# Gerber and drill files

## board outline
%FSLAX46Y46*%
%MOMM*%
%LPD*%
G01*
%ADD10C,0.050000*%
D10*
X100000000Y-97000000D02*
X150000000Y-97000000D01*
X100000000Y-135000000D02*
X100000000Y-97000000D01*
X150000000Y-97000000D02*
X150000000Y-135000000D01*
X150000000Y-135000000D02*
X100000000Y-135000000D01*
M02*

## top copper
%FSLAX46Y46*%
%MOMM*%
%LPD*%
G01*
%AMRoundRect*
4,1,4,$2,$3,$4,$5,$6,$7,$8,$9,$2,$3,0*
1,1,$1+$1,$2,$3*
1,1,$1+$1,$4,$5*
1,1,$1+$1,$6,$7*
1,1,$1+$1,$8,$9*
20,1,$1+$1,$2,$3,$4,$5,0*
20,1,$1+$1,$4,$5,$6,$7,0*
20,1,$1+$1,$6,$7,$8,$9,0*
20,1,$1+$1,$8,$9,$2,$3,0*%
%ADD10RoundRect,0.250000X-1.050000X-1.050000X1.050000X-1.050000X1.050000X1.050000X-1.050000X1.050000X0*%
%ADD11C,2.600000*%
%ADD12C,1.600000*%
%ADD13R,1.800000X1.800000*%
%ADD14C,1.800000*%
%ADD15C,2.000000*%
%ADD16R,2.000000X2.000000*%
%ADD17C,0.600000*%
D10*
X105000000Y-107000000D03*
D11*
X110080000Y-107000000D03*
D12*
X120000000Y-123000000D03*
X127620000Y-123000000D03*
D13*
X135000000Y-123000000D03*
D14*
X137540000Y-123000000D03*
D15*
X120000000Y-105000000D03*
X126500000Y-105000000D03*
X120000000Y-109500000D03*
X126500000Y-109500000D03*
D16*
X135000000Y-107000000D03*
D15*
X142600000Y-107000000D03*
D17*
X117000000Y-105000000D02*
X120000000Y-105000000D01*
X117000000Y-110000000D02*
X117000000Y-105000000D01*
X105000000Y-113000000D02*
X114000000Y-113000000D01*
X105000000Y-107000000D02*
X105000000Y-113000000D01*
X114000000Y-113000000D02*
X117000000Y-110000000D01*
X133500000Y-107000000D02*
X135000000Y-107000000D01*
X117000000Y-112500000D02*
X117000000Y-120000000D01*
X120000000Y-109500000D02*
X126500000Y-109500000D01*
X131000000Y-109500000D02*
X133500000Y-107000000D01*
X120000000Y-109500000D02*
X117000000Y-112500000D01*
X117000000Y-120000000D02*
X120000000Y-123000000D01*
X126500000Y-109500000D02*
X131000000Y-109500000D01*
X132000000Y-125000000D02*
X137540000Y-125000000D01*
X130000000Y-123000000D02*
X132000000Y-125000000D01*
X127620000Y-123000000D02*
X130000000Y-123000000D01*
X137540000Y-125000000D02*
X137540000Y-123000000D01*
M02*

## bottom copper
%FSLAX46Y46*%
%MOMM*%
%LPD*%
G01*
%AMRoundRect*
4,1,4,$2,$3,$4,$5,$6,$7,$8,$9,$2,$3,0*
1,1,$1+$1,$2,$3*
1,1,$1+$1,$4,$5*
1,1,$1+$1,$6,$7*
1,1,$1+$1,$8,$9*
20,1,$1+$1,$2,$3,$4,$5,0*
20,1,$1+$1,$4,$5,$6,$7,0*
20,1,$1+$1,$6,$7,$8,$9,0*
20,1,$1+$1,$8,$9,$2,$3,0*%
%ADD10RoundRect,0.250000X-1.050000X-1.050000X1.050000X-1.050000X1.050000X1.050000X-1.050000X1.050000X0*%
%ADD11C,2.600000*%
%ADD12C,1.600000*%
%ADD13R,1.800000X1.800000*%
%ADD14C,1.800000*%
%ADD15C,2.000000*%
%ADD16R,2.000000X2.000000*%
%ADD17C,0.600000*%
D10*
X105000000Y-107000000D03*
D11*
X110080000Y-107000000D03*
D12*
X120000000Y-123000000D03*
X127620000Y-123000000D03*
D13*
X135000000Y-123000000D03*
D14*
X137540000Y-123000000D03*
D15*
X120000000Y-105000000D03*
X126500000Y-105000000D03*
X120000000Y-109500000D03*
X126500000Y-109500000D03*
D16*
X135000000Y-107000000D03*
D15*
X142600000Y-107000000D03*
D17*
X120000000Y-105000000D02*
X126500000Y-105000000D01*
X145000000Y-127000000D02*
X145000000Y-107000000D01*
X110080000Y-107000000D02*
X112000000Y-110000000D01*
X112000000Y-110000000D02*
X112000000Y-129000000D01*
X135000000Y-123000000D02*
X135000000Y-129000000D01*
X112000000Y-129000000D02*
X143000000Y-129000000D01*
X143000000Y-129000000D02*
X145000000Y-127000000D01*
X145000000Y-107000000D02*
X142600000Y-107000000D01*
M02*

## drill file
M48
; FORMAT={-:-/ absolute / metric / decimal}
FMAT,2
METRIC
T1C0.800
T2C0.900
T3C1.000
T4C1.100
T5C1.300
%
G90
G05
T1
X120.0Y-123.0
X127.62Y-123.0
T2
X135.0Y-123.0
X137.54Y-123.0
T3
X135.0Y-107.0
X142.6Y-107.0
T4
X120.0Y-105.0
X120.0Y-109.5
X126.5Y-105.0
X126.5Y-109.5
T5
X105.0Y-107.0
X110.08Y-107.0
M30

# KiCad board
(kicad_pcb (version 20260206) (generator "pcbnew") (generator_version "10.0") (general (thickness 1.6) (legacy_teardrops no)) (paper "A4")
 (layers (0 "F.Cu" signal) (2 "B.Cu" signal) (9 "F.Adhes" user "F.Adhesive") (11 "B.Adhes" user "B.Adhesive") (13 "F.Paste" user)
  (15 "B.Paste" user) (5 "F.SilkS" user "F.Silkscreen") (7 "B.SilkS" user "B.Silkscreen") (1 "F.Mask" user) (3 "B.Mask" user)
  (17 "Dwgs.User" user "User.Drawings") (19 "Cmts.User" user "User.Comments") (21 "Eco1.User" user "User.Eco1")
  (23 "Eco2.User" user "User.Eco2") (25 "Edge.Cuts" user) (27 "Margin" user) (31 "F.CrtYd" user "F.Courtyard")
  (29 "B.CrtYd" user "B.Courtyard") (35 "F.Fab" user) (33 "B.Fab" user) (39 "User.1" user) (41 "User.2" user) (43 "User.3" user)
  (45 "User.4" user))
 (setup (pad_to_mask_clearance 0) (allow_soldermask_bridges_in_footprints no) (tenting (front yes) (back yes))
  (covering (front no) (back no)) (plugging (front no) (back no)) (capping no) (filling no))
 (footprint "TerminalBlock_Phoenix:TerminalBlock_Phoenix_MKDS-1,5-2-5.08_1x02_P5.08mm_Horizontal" (layer "F.Cu") (at 105 107)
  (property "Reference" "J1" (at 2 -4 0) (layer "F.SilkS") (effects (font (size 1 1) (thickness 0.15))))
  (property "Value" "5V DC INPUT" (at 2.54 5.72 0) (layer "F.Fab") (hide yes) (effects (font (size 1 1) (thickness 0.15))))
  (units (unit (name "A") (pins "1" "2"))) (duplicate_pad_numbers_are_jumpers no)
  (pad "1" thru_hole roundrect (at 0 0) (size 2.6 2.6) (drill 1.3) (layers "*.Cu" "*.Mask") (remove_unused_layers no)
   (roundrect_rratio 0.096154) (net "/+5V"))
  (pad "2" thru_hole circle (at 5.08 0) (size 2.6 2.6) (drill 1.3) (layers "*.Cu" "*.Mask") (remove_unused_layers no) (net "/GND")))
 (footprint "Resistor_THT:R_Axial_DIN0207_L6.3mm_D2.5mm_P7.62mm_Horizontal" (layer "F.Cu") (at 120 123)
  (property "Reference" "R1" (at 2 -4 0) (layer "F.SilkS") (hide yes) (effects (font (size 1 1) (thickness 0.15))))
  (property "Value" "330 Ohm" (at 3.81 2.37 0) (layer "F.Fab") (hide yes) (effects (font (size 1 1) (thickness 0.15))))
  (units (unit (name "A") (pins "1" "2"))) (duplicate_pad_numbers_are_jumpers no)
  (pad "1" thru_hole circle (at 0 0) (size 1.6 1.6) (drill 0.8) (layers "*.Cu" "*.Mask") (remove_unused_layers no) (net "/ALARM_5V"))
  (pad "2" thru_hole circle (at 7.62 0) (size 1.6 1.6) (drill 0.8) (layers "*.Cu" "*.Mask") (remove_unused_layers no) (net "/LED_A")))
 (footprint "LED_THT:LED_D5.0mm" (layer "F.Cu") (at 135 123)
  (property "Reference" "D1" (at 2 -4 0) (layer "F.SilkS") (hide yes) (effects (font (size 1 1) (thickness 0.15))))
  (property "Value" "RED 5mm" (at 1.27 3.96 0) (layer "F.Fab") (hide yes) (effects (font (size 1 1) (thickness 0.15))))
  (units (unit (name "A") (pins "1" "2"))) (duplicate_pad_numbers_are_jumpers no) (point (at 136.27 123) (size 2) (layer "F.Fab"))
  (pad "1" thru_hole rect (at 0 0) (size 1.8 1.8) (drill 0.9) (layers "*.Cu" "*.Mask") (remove_unused_layers no) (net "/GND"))
  (pad "2" thru_hole circle (at 2.54 0) (size 1.8 1.8) (drill 0.9) (layers "*.Cu" "*.Mask") (remove_unused_layers no) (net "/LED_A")))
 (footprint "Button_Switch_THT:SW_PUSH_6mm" (layer "F.Cu") (at 120 105)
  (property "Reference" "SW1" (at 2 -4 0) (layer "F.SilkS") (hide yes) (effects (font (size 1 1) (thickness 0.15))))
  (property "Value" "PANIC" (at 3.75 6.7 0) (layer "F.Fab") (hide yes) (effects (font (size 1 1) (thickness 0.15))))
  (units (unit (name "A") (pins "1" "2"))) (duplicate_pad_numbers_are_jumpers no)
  (pad "1" thru_hole circle (at 0 0 90) (size 2 2) (drill 1.1) (layers "*.Cu" "*.Mask") (remove_unused_layers no) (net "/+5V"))
  (pad "1" thru_hole circle (at 6.5 0 90) (size 2 2) (drill 1.1) (layers "*.Cu" "*.Mask") (remove_unused_layers no) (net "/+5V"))
  (pad "2" thru_hole circle (at 0 4.5 90) (size 2 2) (drill 1.1) (layers "*.Cu" "*.Mask") (remove_unused_layers no) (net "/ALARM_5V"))
  (pad "2" thru_hole circle (at 6.5 4.5 90) (size 2 2) (drill 1.1) (layers "*.Cu" "*.Mask") (remove_unused_layers no) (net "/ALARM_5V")))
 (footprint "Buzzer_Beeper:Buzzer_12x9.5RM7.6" (layer "F.Cu") (at 135 107)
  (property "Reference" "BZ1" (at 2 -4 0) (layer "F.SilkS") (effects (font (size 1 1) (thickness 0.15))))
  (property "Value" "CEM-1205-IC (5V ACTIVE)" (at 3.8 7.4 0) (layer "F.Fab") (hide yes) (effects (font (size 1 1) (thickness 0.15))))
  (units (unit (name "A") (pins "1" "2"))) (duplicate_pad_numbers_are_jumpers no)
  (pad "1" thru_hole rect (at 0 0) (size 2 2) (drill 1) (layers "*.Cu" "*.Mask") (remove_unused_layers no) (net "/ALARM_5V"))
  (pad "2" thru_hole circle (at 7.6 0) (size 2 2) (drill 1) (layers "*.Cu" "*.Mask") (remove_unused_layers no) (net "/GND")))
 (gr_line (start 100 97) (end 150 97) (stroke (width 0.05) (type default)) (layer "Edge.Cuts"))
 (gr_line (start 100 135) (end 100 97) (stroke (width 0.05) (type default)) (layer "Edge.Cuts"))
 (gr_line (start 150 97) (end 150 135) (stroke (width 0.05) (type default)) (layer "Edge.Cuts"))
 (gr_line (start 150 135) (end 100 135) (stroke (width 0.05) (type default)) (layer "Edge.Cuts"))
 (segment (start 117 105) (end 120 105) (width 0.6) (layer "F.Cu") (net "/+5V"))
 (segment (start 117 110) (end 117 105) (width 0.6) (layer "F.Cu") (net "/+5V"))
 (segment (start 105 113) (end 114 113) (width 0.6) (layer "F.Cu") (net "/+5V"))
 (segment (start 105 107) (end 105 113) (width 0.6) (layer "F.Cu") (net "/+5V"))
 (segment (start 114 113) (end 117 110) (width 0.6) (layer "F.Cu") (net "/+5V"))
 (segment (start 120 105) (end 126.5 105) (width 0.6) (layer "B.Cu") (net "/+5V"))
 (segment (start 145 127) (end 145 107) (width 0.6) (layer "B.Cu") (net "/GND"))
 (segment (start 110.08 107) (end 112 110) (width 0.6) (layer "B.Cu") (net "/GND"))
 (segment (start 112 110) (end 112 129) (width 0.6) (layer "B.Cu") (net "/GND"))
 (segment (start 135 123) (end 135 129) (width 0.6) (layer "B.Cu") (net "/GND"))
 (segment (start 112 129) (end 143 129) (width 0.6) (layer "B.Cu") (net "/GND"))
 (segment (start 143 129) (end 145 127) (width 0.6) (layer "B.Cu") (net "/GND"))
 (segment (start 145 107) (end 142.6 107) (width 0.6) (layer "B.Cu") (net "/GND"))
 (segment (start 133.5 107) (end 135 107) (width 0.6) (layer "F.Cu") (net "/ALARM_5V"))
 (segment (start 117 112.5) (end 117 120) (width 0.6) (layer "F.Cu") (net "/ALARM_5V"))
 (segment (start 120 109.5) (end 126.5 109.5) (width 0.6) (layer "F.Cu") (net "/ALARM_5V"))
 (segment (start 131 109.5) (end 133.5 107) (width 0.6) (layer "F.Cu") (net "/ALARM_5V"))
 (segment (start 120 109.5) (end 117 112.5) (width 0.6) (layer "F.Cu") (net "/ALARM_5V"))
 (segment (start 117 120) (end 120 123) (width 0.6) (layer "F.Cu") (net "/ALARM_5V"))
 (segment (start 126.5 109.5) (end 131 109.5) (width 0.6) (layer "F.Cu") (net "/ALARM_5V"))
 (segment (start 132 125) (end 137.54 125) (width 0.6) (layer "F.Cu") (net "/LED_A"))
 (segment (start 130 123) (end 132 125) (width 0.6) (layer "F.Cu") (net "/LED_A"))
 (segment (start 127.62 123) (end 130 123) (width 0.6) (layer "F.Cu") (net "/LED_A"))
 (segment (start 137.54 125) (end 137.54 123) (width 0.6) (layer "F.Cu") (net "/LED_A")))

